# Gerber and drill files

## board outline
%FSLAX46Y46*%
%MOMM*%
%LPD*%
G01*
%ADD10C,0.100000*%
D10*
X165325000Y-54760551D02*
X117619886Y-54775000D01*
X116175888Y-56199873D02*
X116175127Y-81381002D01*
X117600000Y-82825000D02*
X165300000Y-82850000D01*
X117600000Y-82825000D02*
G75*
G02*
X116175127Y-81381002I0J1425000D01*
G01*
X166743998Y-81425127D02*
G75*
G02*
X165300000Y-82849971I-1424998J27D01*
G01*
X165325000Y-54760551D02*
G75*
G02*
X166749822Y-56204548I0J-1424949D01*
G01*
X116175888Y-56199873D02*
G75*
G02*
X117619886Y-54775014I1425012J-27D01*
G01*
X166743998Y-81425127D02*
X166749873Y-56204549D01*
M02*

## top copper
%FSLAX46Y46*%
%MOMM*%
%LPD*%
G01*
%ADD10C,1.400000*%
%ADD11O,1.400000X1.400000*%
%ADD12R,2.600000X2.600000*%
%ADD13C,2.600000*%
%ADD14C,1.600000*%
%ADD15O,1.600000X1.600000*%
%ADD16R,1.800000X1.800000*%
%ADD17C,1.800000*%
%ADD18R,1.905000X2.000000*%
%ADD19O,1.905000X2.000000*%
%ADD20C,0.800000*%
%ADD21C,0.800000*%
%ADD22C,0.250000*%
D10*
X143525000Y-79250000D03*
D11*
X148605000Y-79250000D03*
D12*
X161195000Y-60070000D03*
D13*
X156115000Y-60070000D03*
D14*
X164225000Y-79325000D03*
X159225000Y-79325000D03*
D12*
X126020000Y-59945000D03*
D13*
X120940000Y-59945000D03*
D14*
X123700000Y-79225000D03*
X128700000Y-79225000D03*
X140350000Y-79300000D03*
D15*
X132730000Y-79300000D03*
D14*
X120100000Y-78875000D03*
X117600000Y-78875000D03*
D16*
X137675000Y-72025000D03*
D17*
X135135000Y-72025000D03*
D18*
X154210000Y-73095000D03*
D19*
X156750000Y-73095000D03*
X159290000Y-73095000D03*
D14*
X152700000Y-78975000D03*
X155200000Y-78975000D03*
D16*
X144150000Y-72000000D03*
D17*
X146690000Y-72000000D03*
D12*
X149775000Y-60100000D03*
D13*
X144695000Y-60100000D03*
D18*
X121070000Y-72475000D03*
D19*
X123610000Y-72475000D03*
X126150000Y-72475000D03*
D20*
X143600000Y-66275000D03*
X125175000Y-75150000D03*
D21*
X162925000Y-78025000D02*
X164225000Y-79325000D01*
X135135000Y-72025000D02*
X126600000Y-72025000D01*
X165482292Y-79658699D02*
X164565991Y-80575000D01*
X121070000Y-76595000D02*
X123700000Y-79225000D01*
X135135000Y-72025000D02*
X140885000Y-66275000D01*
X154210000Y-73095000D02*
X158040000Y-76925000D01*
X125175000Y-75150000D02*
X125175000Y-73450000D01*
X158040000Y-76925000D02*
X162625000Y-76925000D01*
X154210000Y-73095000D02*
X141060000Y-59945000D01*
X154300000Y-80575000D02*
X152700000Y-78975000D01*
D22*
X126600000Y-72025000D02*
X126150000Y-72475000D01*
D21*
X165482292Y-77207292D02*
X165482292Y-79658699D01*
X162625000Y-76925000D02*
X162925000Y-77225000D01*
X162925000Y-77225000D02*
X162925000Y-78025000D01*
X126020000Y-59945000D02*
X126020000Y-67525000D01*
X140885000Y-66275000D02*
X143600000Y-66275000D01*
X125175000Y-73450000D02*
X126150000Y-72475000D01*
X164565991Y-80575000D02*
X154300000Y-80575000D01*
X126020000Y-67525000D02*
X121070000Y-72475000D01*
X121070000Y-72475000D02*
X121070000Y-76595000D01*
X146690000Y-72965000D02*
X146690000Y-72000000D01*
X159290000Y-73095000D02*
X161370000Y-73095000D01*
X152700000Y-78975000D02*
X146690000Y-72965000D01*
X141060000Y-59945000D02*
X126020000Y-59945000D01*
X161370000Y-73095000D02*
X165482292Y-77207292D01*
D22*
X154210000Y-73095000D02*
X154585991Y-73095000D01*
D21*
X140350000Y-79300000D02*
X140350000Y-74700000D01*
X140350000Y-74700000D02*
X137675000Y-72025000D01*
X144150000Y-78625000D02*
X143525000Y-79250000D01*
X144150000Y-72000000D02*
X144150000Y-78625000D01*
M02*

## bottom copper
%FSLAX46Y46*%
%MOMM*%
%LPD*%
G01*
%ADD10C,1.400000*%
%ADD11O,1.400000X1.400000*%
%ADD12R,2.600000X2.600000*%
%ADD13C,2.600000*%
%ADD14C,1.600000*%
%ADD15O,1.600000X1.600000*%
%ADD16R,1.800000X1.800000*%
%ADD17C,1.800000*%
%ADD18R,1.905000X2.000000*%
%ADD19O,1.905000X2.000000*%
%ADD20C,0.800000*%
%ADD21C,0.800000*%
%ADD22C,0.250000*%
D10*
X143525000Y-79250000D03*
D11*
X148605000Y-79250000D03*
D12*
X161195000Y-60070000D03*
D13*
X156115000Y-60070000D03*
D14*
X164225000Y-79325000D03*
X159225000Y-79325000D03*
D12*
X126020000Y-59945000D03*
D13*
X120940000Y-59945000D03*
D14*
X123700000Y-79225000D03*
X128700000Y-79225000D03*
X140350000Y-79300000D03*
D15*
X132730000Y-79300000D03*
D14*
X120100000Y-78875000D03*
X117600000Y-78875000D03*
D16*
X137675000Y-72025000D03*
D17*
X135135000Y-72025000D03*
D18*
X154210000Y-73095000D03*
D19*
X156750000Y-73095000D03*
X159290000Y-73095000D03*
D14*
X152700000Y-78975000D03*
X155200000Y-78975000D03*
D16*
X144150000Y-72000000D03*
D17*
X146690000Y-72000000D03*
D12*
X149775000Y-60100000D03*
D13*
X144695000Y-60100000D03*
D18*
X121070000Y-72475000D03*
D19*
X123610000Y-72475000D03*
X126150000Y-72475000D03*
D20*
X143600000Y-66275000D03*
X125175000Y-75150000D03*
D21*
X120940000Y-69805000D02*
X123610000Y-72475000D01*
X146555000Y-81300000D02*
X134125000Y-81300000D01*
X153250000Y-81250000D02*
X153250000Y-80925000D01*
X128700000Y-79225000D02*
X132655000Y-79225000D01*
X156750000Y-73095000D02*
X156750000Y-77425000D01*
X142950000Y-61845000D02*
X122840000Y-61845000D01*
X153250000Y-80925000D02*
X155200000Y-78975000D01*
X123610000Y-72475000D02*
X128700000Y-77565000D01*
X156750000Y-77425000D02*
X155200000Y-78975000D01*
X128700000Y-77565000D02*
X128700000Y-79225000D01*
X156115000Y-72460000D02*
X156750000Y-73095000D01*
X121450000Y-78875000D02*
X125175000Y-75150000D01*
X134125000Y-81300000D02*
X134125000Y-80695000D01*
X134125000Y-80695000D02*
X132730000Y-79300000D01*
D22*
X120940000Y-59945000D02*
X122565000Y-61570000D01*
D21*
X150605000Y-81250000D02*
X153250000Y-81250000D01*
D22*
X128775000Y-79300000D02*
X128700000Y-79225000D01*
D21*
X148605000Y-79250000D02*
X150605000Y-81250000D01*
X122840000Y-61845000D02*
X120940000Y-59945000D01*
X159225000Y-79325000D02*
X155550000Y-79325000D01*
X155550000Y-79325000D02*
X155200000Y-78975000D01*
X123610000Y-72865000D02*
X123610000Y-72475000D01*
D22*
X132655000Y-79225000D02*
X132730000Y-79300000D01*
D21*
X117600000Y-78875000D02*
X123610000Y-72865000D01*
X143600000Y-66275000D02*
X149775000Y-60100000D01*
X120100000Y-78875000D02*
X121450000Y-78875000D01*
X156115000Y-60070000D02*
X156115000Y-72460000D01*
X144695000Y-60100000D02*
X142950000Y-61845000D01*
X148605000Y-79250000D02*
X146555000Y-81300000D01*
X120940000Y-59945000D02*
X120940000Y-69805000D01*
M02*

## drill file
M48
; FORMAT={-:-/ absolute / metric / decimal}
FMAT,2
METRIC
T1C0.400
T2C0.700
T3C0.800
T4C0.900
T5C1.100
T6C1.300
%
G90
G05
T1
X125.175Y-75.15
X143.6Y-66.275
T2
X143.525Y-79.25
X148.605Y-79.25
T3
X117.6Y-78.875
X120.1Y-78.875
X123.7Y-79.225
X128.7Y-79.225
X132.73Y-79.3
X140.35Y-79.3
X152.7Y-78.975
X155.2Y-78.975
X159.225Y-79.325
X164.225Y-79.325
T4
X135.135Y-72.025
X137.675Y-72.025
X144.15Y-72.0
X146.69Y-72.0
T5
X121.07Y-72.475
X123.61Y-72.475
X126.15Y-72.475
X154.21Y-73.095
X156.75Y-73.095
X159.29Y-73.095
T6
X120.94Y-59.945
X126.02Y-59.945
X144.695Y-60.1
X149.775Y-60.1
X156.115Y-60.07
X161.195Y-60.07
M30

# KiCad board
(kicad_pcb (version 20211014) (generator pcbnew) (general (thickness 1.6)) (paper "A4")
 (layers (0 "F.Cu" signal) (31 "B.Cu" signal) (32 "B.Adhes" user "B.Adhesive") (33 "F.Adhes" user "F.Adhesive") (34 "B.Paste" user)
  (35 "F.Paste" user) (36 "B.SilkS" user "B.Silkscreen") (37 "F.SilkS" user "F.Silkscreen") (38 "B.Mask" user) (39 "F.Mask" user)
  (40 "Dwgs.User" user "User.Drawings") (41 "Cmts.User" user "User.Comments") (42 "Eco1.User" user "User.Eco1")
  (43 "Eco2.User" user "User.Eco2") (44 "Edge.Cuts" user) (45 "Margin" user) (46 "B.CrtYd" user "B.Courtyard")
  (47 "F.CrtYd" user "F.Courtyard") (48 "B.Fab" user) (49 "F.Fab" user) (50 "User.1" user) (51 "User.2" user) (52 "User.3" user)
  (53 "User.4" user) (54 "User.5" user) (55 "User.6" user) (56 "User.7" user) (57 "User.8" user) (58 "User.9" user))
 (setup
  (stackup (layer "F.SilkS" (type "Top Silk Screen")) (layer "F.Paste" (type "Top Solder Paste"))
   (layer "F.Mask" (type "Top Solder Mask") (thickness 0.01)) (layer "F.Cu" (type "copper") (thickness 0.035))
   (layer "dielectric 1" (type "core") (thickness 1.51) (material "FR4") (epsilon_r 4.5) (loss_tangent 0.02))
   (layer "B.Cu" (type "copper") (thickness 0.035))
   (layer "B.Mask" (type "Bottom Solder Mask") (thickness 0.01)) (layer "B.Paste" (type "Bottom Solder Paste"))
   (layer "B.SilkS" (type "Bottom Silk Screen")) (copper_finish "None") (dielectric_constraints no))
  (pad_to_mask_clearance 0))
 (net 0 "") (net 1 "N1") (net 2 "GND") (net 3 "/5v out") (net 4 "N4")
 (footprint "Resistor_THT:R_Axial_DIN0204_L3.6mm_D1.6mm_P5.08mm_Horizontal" (layer "F.Cu") (at 143.525 79.25)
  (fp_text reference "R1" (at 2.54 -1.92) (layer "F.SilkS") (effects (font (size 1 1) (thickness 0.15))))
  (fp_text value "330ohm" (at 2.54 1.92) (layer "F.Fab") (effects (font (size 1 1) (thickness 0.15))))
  (pad "1" thru_hole circle (at 0 0) (size 1.4 1.4) (drill 0.7) (layers *.Cu *.Mask) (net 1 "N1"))
  (pad "2" thru_hole oval (at 5.08 0) (size 1.4 1.4) (drill 0.7) (layers *.Cu *.Mask) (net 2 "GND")))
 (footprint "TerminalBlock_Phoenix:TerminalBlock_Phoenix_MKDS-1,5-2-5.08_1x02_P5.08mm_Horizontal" (layer "F.Cu") (at 161.195 60.07 180)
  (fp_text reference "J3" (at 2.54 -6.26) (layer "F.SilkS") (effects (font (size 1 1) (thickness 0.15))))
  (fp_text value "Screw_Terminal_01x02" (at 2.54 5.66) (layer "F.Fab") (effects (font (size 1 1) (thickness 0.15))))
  (pad "1" thru_hole rect (at 0 0 180) (size 2.6 2.6) (drill 1.3) (layers *.Cu *.Mask) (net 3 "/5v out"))
  (pad "2" thru_hole circle (at 5.08 0 180) (size 2.6 2.6) (drill 1.3) (layers *.Cu *.Mask) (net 2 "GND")))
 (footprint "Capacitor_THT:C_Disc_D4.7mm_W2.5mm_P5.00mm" (layer "F.Cu") (at 164.225 79.325 180)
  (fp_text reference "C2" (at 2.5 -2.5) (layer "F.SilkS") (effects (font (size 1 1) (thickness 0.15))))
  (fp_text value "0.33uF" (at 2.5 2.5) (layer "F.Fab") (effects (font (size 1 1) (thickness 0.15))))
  (pad "1" thru_hole circle (at 0 0 180) (size 1.6 1.6) (drill 0.8) (layers *.Cu *.Mask) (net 2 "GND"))
  (pad "2" thru_hole circle (at 5 0 180) (size 1.6 1.6) (drill 0.8) (layers *.Cu *.Mask) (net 2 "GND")))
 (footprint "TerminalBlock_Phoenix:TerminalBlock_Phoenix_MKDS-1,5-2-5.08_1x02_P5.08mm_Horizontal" (layer "F.Cu") (at 126.02 59.945 180)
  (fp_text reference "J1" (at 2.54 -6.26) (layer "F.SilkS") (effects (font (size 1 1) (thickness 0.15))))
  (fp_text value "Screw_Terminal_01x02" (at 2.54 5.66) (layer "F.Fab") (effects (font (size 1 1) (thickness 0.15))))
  (pad "1" thru_hole rect (at 0 0 180) (size 2.6 2.6) (drill 1.3) (layers *.Cu *.Mask) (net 2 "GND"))
  (pad "2" thru_hole circle (at 5.08 0 180) (size 2.6 2.6) (drill 1.3) (layers *.Cu *.Mask) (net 2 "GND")))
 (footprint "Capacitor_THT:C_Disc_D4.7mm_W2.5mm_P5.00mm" (layer "F.Cu") (at 123.7 79.225)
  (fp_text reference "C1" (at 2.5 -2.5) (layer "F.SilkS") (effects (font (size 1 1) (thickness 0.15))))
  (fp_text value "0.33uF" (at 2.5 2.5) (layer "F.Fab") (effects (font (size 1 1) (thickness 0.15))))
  (pad "1" thru_hole circle (at 0 0) (size 1.6 1.6) (drill 0.8) (layers *.Cu *.Mask) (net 2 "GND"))
  (pad "2" thru_hole circle (at 5 0) (size 1.6 1.6) (drill 0.8) (layers *.Cu *.Mask) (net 2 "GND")))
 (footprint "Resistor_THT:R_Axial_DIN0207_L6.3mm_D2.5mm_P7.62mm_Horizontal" (layer "F.Cu") (at 140.35 79.3 180)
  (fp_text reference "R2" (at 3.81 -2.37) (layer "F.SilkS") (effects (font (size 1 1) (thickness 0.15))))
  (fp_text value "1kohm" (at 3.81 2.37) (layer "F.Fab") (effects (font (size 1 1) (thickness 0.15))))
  (pad "1" thru_hole circle (at 0 0 180) (size 1.6 1.6) (drill 0.8) (layers *.Cu *.Mask) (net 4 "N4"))
  (pad "2" thru_hole oval (at 7.62 0 180) (size 1.6 1.6) (drill 0.8) (layers *.Cu *.Mask) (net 2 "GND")))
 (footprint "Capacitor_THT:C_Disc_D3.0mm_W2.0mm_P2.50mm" (layer "F.Cu") (at 120.1 78.875 180)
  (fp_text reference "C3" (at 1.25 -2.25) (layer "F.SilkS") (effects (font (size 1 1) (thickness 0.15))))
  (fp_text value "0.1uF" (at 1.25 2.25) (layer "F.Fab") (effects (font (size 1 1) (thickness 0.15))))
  (pad "1" thru_hole circle (at 0 0 180) (size 1.6 1.6) (drill 0.8) (layers *.Cu *.Mask) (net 2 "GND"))
  (pad "2" thru_hole circle (at 2.5 0 180) (size 1.6 1.6) (drill 0.8) (layers *.Cu *.Mask) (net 2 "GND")))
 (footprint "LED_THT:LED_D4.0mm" (layer "F.Cu") (at 137.675 72.025 180)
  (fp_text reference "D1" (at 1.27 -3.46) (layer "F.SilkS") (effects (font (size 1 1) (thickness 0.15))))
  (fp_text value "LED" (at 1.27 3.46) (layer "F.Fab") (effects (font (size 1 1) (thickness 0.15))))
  (pad "1" thru_hole rect (at 0 0 180) (size 1.8 1.8) (drill 0.9) (layers *.Cu *.Mask) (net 4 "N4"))
  (pad "2" thru_hole circle (at 2.54 0 180) (size 1.8 1.8) (drill 0.9) (layers *.Cu *.Mask) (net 2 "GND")))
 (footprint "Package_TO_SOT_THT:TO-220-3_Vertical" (layer "F.Cu") (at 154.21 73.095)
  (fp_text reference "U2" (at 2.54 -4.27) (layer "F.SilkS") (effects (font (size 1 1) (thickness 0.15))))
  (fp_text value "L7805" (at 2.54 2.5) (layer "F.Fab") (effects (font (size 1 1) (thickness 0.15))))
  (pad "1" thru_hole rect (at 0 0) (size 1.905 2) (drill 1.1) (layers *.Cu *.Mask) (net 2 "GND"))
  (pad "2" thru_hole oval (at 2.54 0) (size 1.905 2) (drill 1.1) (layers *.Cu *.Mask) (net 2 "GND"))
  (pad "3" thru_hole oval (at 5.08 0) (size 1.905 2) (drill 1.1) (layers *.Cu *.Mask) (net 2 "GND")))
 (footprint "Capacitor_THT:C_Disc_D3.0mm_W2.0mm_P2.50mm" (layer "F.Cu") (at 152.7 78.975)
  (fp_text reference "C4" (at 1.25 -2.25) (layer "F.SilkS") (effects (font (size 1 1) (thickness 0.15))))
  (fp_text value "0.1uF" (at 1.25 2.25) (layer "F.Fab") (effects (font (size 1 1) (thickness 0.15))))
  (pad "1" thru_hole circle (at 0 0) (size 1.6 1.6) (drill 0.8) (layers *.Cu *.Mask) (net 2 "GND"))
  (pad "2" thru_hole circle (at 2.5 0) (size 1.6 1.6) (drill 0.8) (layers *.Cu *.Mask) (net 2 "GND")))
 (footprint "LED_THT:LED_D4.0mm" (layer "F.Cu") (at 144.15 72)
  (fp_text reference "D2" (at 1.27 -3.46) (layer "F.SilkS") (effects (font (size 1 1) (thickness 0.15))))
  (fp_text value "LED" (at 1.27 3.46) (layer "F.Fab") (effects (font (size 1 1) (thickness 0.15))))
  (pad "1" thru_hole rect (at 0 0) (size 1.8 1.8) (drill 0.9) (layers *.Cu *.Mask) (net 1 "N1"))
  (pad "2" thru_hole circle (at 2.54 0) (size 1.8 1.8) (drill 0.9) (layers *.Cu *.Mask) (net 2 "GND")))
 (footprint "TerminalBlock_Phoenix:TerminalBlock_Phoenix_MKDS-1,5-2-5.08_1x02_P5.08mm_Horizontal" (layer "F.Cu") (at 149.775 60.1 180)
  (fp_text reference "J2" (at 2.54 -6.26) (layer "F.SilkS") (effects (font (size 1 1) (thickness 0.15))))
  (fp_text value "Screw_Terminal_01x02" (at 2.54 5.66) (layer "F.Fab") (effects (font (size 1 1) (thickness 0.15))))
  (pad "1" thru_hole rect (at 0 0 180) (size 2.6 2.6) (drill 1.3) (layers *.Cu *.Mask) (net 2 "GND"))
  (pad "2" thru_hole circle (at 5.08 0 180) (size 2.6 2.6) (drill 1.3) (layers *.Cu *.Mask) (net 2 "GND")))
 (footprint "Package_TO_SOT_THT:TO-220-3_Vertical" (layer "F.Cu") (at 121.07 72.475)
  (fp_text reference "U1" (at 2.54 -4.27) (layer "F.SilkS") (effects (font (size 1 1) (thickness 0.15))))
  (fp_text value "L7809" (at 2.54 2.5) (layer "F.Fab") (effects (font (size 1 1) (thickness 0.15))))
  (pad "1" thru_hole rect (at 0 0) (size 1.905 2) (drill 1.1) (layers *.Cu *.Mask) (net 2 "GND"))
  (pad "2" thru_hole oval (at 2.54 0) (size 1.905 2) (drill 1.1) (layers *.Cu *.Mask) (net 2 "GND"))
  (pad "3" thru_hole oval (at 5.08 0) (size 1.905 2) (drill 1.1) (layers *.Cu *.Mask) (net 2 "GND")))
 (gr_line (start 165.325 54.760551) (end 117.619886 54.775) (layer "Edge.Cuts") (width 0.1))
 (gr_line (start 116.175888 56.199873) (end 116.175127 81.381002) (layer "Edge.Cuts") (width 0.1))
 (gr_line (start 117.6 82.825) (end 165.3 82.85) (layer "Edge.Cuts") (width 0.1))
 (gr_arc (start 117.6 82.825) (mid 116.585678 82.400888) (end 116.175127 81.381002) (layer "Edge.Cuts") (width 0.1))
 (gr_arc (start 166.743998 81.425127) (mid 166.319877 82.439435) (end 165.3 82.85) (layer "Edge.Cuts") (width 0.1))
 (gr_arc (start 165.325 54.760551) (mid 166.339322 55.184663) (end 166.749873 56.204549) (layer "Edge.Cuts") (width 0.1))
 (gr_arc (start 116.175888 56.199873) (mid 116.6 55.185551) (end 117.619886 54.775) (layer "Edge.Cuts") (width 0.1))
 (gr_line (start 166.743998 81.425127) (end 166.749873 56.204549) (layer "Edge.Cuts") (width 0.1))
 (segment (start 162.925 78.025) (end 164.225 79.325) (width 0.8) (layer "F.Cu") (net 2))
 (segment (start 135.135 72.025) (end 126.6 72.025) (width 0.8) (layer "F.Cu") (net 2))
 (segment (start 165.482292 79.658699) (end 164.565991 80.575) (width 0.8) (layer "F.Cu") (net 2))
 (segment (start 121.07 76.595) (end 123.7 79.225) (width 0.8) (layer "F.Cu") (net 2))
 (segment (start 135.135 72.025) (end 140.885 66.275) (width 0.8) (layer "F.Cu") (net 2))
 (segment (start 154.21 73.095) (end 158.04 76.925) (width 0.8) (layer "F.Cu") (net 2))
 (segment (start 125.175 75.15) (end 125.175 73.45) (width 0.8) (layer "F.Cu") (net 2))
 (segment (start 158.04 76.925) (end 162.625 76.925) (width 0.8) (layer "F.Cu") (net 2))
 (segment (start 154.21 73.095) (end 141.06 59.945) (width 0.8) (layer "F.Cu") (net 2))
 (segment (start 154.3 80.575) (end 152.7 78.975) (width 0.8) (layer "F.Cu") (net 2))
 (segment (start 126.6 72.025) (end 126.15 72.475) (width 0.25) (layer "F.Cu") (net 2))
 (segment (start 165.482292 77.207292) (end 165.482292 79.658699) (width 0.8) (layer "F.Cu") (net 2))
 (segment (start 162.625 76.925) (end 162.925 77.225) (width 0.8) (layer "F.Cu") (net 2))
 (segment (start 162.925 77.225) (end 162.925 78.025) (width 0.8) (layer "F.Cu") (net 2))
 (segment (start 126.02 59.945) (end 126.02 67.525) (width 0.8) (layer "F.Cu") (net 2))
 (segment (start 140.885 66.275) (end 143.6 66.275) (width 0.8) (layer "F.Cu") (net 2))
 (segment (start 125.175 73.45) (end 126.15 72.475) (width 0.8) (layer "F.Cu") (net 2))
 (segment (start 164.565991 80.575) (end 154.3 80.575) (width 0.8) (layer "F.Cu") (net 2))
 (segment (start 126.02 67.525) (end 121.07 72.475) (width 0.8) (layer "F.Cu") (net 2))
 (segment (start 121.07 72.475) (end 121.07 76.595) (width 0.8) (layer "F.Cu") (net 2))
 (segment (start 146.69 72.965) (end 146.69 72) (width 0.8) (layer "F.Cu") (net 2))
 (segment (start 159.29 73.095) (end 161.37 73.095) (width 0.8) (layer "F.Cu") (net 2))
 (segment (start 152.7 78.975) (end 146.69 72.965) (width 0.8) (layer "F.Cu") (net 2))
 (segment (start 141.06 59.945) (end 126.02 59.945) (width 0.8) (layer "F.Cu") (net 2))
 (segment (start 161.37 73.095) (end 165.482292 77.207292) (width 0.8) (layer "F.Cu") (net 2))
 (segment (start 154.21 73.095) (end 154.585991 73.095) (width 0.25) (layer "F.Cu") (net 2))
 (via (at 143.6 66.275) (size 0.8) (drill 0.4) (layers "F.Cu" "B.Cu") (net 2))
 (via (at 125.175 75.15) (size 0.8) (drill 0.4) (layers "F.Cu" "B.Cu") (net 2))
 (segment (start 120.94 69.805) (end 123.61 72.475) (width 0.8) (layer "B.Cu") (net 2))
 (segment (start 146.555 81.3) (end 134.125 81.3) (width 0.8) (layer "B.Cu") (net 2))
 (segment (start 153.25 81.25) (end 153.25 80.925) (width 0.8) (layer "B.Cu") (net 2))
 (segment (start 128.7 79.225) (end 132.655 79.225) (width 0.8) (layer "B.Cu") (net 2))
 (segment (start 156.75 73.095) (end 156.75 77.425) (width 0.8) (layer "B.Cu") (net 2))
 (segment (start 142.95 61.845) (end 122.84 61.845) (width 0.8) (layer "B.Cu") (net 2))
 (segment (start 153.25 80.925) (end 155.2 78.975) (width 0.8) (layer "B.Cu") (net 2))
 (segment (start 123.61 72.475) (end 128.7 77.565) (width 0.8) (layer "B.Cu") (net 2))
 (segment (start 156.75 77.425) (end 155.2 78.975) (width 0.8) (layer "B.Cu") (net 2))
 (segment (start 128.7 77.565) (end 128.7 79.225) (width 0.8) (layer "B.Cu") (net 2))
 (segment (start 156.115 72.46) (end 156.75 73.095) (width 0.8) (layer "B.Cu") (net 2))
 (segment (start 121.45 78.875) (end 125.175 75.15) (width 0.8) (layer "B.Cu") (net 2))
 (segment (start 134.125 81.3) (end 134.125 80.695) (width 0.8) (layer "B.Cu") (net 2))
 (segment (start 134.125 80.695) (end 132.73 79.3) (width 0.8) (layer "B.Cu") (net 2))
 (segment (start 120.94 59.945) (end 122.565 61.57) (width 0.25) (layer "B.Cu") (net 2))
 (segment (start 150.605 81.25) (end 153.25 81.25) (width 0.8) (layer "B.Cu") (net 2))
 (segment (start 128.775 79.3) (end 128.7 79.225) (width 0.25) (layer "B.Cu") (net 2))
 (segment (start 148.605 79.25) (end 150.605 81.25) (width 0.8) (layer "B.Cu") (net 2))
 (segment (start 122.84 61.845) (end 120.94 59.945) (width 0.8) (layer "B.Cu") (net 2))
 (segment (start 159.225 79.325) (end 155.55 79.325) (width 0.8) (layer "B.Cu") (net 2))
 (segment (start 155.55 79.325) (end 155.2 78.975) (width 0.8) (layer "B.Cu") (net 2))
 (segment (start 123.61 72.865) (end 123.61 72.475) (width 0.8) (layer "B.Cu") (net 2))
 (segment (start 132.655 79.225) (end 132.73 79.3) (width 0.25) (layer "B.Cu") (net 2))
 (segment (start 117.6 78.875) (end 123.61 72.865) (width 0.8) (layer "B.Cu") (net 2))
 (segment (start 143.6 66.275) (end 149.775 60.1) (width 0.8) (layer "B.Cu") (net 2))
 (segment (start 120.1 78.875) (end 121.45 78.875) (width 0.8) (layer "B.Cu") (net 2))
 (segment (start 156.115 60.07) (end 156.115 72.46) (width 0.8) (layer "B.Cu") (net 2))
 (segment (start 144.695 60.1) (end 142.95 61.845) (width 0.8) (layer "B.Cu") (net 2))
 (segment (start 148.605 79.25) (end 146.555 81.3) (width 0.8) (layer "B.Cu") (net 2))
 (segment (start 120.94 59.945) (end 120.94 69.805) (width 0.8) (layer "B.Cu") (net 2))
 (segment (start 140.35 79.3) (end 140.35 74.7) (width 0.8) (layer "F.Cu") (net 4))
 (segment (start 140.35 74.7) (end 137.675 72.025) (width 0.8) (layer "F.Cu") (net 4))
 (segment (start 144.15 78.625) (end 143.525 79.25) (width 0.8) (layer "F.Cu") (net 1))
 (segment (start 144.15 72) (end 144.15 78.625) (width 0.8) (layer "F.Cu") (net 1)))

